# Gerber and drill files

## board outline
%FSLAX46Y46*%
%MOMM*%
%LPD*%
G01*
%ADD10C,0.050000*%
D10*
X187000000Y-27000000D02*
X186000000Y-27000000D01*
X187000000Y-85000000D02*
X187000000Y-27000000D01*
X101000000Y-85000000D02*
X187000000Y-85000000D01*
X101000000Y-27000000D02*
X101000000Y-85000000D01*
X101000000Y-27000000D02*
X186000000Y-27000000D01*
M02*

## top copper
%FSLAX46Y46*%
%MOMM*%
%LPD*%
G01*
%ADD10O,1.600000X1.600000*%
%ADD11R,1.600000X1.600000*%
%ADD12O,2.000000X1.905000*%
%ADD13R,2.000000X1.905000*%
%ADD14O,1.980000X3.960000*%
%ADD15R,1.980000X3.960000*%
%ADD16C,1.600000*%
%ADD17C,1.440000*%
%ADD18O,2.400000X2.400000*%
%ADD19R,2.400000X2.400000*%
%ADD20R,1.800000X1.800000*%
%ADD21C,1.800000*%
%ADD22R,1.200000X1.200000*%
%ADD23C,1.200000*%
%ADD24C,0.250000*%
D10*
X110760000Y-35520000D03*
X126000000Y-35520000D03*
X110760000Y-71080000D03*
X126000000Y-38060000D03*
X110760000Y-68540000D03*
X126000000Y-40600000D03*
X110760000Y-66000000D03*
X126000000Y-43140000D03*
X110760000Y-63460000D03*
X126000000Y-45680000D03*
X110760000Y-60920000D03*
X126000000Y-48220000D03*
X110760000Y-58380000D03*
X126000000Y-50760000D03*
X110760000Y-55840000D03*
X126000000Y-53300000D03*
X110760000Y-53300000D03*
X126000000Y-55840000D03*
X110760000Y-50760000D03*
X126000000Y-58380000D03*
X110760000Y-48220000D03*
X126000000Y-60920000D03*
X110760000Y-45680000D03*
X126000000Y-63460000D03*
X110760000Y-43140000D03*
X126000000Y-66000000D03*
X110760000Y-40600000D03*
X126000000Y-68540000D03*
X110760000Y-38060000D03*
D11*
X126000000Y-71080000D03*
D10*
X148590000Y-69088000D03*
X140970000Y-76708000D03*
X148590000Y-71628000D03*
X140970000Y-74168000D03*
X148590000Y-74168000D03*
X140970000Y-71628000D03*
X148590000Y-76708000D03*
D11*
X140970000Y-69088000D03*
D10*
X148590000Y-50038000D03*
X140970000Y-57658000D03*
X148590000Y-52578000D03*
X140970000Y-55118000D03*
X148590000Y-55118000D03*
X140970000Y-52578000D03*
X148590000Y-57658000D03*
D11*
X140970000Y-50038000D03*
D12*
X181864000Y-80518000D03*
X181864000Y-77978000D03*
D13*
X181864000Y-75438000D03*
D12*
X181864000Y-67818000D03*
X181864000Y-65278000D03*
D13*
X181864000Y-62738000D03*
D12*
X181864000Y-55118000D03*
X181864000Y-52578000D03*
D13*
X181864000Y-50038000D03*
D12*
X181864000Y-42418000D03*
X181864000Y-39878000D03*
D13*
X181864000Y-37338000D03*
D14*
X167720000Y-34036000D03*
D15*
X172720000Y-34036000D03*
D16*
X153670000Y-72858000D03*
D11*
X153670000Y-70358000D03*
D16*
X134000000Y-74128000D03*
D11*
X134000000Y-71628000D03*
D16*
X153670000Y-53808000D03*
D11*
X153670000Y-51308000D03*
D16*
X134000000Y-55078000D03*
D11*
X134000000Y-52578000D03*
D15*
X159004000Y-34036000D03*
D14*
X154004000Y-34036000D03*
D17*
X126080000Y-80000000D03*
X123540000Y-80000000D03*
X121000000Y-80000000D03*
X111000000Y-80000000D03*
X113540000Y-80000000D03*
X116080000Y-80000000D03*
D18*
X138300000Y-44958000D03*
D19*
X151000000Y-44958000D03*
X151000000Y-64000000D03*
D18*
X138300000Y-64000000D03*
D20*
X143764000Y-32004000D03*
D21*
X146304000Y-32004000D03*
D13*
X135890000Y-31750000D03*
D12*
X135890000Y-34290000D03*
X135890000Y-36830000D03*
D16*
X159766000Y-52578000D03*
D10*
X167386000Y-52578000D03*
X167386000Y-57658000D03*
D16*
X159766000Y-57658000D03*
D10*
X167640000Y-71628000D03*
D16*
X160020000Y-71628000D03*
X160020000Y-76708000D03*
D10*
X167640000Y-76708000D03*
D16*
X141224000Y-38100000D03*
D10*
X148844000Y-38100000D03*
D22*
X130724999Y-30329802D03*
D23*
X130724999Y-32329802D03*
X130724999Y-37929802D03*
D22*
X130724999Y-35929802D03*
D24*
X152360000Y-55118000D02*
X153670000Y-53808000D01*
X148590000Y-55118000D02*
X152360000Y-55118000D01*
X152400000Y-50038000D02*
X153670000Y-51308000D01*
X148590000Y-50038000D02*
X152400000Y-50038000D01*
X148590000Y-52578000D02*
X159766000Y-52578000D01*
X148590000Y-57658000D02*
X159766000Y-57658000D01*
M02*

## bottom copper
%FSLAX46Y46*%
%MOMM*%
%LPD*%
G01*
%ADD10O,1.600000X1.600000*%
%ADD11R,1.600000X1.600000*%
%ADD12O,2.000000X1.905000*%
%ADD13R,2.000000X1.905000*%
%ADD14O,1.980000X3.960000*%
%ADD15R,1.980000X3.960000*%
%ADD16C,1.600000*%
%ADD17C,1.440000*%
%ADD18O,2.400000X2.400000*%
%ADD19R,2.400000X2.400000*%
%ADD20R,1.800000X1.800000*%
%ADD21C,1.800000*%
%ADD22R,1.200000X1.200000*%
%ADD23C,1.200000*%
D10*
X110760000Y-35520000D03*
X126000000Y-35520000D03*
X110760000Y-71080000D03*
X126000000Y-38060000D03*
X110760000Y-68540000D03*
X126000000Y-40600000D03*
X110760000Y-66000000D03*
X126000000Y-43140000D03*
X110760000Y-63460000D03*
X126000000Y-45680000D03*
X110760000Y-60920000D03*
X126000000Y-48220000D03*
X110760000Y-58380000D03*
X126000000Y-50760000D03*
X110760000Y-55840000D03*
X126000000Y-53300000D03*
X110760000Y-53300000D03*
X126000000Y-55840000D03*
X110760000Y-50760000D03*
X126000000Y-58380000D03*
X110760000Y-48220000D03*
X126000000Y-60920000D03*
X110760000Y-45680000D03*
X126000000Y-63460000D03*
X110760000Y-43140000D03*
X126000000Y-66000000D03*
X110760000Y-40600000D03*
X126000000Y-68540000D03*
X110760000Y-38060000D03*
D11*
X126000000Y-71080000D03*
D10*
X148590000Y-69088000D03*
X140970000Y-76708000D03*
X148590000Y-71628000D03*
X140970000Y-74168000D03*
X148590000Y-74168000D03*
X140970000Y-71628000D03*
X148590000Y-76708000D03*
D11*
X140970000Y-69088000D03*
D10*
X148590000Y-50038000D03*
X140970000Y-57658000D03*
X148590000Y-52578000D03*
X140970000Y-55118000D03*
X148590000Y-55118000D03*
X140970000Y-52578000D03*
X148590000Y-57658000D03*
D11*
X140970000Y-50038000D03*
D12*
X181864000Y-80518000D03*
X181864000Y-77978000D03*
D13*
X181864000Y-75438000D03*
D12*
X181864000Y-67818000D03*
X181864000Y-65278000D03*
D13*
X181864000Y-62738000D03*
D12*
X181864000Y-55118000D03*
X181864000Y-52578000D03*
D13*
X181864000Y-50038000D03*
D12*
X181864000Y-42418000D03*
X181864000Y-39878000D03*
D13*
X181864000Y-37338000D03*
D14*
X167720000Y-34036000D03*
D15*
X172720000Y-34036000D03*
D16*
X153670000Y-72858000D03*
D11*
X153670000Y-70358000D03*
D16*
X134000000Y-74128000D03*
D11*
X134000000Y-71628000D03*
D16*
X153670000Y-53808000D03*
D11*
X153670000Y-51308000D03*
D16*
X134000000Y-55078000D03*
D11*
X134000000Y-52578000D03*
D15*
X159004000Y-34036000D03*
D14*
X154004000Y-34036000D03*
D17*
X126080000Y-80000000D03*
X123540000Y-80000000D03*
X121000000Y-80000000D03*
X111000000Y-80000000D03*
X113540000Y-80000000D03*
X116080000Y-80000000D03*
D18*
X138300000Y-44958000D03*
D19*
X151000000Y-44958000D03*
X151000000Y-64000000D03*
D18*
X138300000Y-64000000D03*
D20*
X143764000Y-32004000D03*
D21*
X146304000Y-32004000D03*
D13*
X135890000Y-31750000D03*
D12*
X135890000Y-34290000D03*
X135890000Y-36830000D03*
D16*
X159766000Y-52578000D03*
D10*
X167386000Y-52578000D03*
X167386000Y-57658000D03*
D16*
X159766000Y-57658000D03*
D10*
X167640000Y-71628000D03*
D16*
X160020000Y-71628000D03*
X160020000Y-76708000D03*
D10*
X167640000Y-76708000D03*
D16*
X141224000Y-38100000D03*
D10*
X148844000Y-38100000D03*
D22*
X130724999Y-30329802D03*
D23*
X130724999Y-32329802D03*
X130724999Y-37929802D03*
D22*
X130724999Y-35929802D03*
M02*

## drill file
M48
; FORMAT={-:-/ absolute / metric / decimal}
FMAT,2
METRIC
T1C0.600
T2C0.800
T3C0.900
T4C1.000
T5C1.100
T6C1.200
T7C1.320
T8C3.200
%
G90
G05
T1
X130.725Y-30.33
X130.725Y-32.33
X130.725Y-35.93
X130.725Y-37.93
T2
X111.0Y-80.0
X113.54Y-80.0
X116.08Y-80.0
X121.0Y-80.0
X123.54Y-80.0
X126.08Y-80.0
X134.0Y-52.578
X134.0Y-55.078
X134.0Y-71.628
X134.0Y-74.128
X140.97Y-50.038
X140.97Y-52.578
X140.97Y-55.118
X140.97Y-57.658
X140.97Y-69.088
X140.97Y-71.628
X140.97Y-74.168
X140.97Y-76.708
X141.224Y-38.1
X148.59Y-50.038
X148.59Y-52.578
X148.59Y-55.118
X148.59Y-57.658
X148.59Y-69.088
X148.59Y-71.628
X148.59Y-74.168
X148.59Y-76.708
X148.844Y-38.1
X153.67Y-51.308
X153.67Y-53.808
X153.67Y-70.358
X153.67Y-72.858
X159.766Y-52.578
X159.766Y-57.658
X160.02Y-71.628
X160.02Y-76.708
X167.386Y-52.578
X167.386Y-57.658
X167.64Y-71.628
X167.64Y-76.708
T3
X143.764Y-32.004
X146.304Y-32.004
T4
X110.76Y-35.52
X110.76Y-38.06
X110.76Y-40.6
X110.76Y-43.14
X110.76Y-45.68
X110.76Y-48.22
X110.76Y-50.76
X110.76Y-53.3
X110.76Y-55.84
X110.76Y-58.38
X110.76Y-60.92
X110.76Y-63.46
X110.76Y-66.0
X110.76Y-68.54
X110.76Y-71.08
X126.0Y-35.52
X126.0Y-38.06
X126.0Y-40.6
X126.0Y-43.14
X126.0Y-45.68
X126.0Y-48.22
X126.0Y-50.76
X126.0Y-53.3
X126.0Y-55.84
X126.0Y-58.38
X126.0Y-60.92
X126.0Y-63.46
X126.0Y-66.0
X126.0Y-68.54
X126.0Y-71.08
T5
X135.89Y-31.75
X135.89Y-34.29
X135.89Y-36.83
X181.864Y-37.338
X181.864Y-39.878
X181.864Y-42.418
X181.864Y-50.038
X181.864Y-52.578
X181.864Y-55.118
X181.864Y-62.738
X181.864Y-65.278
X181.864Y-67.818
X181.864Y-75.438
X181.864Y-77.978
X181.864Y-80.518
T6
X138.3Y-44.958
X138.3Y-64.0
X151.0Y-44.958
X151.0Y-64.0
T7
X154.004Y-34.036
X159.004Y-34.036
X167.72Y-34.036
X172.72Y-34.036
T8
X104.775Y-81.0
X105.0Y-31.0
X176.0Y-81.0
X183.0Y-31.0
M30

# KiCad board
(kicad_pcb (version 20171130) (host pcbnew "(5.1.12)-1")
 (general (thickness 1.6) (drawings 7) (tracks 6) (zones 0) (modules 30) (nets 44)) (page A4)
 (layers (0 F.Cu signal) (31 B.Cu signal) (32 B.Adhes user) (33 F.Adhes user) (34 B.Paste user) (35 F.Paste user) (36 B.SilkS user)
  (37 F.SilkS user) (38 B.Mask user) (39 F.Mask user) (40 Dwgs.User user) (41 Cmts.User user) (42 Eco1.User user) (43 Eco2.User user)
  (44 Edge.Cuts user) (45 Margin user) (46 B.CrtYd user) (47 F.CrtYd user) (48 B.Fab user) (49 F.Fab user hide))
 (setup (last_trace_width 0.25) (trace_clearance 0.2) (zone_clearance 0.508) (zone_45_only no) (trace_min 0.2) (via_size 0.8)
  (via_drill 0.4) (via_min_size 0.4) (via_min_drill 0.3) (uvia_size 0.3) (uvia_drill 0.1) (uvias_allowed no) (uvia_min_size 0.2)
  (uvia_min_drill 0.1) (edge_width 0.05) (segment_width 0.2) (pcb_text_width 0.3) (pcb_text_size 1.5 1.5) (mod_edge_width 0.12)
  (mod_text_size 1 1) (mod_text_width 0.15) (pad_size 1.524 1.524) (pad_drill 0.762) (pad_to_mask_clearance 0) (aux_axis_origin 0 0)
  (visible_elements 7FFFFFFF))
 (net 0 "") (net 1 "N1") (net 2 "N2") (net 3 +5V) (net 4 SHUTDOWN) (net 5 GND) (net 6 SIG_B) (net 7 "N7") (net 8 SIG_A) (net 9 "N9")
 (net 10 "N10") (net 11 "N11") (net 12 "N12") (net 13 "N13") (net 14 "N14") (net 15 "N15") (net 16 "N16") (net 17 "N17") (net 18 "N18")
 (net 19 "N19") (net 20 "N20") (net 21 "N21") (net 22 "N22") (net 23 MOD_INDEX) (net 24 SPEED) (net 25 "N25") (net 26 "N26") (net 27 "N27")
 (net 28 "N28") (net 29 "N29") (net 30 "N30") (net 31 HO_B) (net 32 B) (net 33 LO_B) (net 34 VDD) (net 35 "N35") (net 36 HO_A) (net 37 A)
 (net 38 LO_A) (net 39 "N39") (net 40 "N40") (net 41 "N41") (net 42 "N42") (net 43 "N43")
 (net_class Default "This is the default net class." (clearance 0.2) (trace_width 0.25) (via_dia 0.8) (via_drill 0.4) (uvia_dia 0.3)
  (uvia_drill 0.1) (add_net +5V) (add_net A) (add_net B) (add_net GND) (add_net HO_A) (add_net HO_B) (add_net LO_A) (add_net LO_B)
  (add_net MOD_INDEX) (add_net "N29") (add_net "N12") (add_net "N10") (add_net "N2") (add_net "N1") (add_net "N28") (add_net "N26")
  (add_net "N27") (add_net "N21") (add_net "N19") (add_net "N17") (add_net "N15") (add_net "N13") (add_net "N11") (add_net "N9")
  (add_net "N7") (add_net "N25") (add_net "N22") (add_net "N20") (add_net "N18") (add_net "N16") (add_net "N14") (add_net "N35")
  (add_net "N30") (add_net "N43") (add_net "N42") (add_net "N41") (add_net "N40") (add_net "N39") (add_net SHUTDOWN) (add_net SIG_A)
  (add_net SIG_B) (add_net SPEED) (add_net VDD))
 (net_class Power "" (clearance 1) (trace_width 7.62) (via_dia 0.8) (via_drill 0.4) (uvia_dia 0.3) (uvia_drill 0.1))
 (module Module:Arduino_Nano (layer F.Cu) (at 126 71.08 180)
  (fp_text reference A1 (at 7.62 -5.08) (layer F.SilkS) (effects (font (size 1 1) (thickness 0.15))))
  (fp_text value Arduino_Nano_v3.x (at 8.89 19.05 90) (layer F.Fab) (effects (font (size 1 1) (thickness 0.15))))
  (pad 16 thru_hole oval (at 15.24 35.56 180) (size 1.6 1.6) (drill 1) (layers *.Cu *.Mask) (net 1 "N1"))
  (pad 15 thru_hole oval (at 0 35.56 180) (size 1.6 1.6) (drill 1) (layers *.Cu *.Mask) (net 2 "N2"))
  (pad 30 thru_hole oval (at 15.24 0 180) (size 1.6 1.6) (drill 1) (layers *.Cu *.Mask) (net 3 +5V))
  (pad 14 thru_hole oval (at 0 33.02 180) (size 1.6 1.6) (drill 1) (layers *.Cu *.Mask) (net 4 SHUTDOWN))
  (pad 29 thru_hole oval (at 15.24 2.54 180) (size 1.6 1.6) (drill 1) (layers *.Cu *.Mask) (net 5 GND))
  (pad 13 thru_hole oval (at 0 30.48 180) (size 1.6 1.6) (drill 1) (layers *.Cu *.Mask) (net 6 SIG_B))
  (pad 28 thru_hole oval (at 15.24 5.08 180) (size 1.6 1.6) (drill 1) (layers *.Cu *.Mask) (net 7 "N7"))
  (pad 12 thru_hole oval (at 0 27.94 180) (size 1.6 1.6) (drill 1) (layers *.Cu *.Mask) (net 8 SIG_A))
  (pad 27 thru_hole oval (at 15.24 7.62 180) (size 1.6 1.6) (drill 1) (layers *.Cu *.Mask) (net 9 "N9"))
  (pad 11 thru_hole oval (at 0 25.4 180) (size 1.6 1.6) (drill 1) (layers *.Cu *.Mask) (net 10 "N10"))
  (pad 26 thru_hole oval (at 15.24 10.16 180) (size 1.6 1.6) (drill 1) (layers *.Cu *.Mask) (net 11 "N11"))
  (pad 10 thru_hole oval (at 0 22.86 180) (size 1.6 1.6) (drill 1) (layers *.Cu *.Mask) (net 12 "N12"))
  (pad 25 thru_hole oval (at 15.24 12.7 180) (size 1.6 1.6) (drill 1) (layers *.Cu *.Mask) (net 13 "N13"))
  (pad 9 thru_hole oval (at 0 20.32 180) (size 1.6 1.6) (drill 1) (layers *.Cu *.Mask) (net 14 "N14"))
  (pad 24 thru_hole oval (at 15.24 15.24 180) (size 1.6 1.6) (drill 1) (layers *.Cu *.Mask) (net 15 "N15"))
  (pad 8 thru_hole oval (at 0 17.78 180) (size 1.6 1.6) (drill 1) (layers *.Cu *.Mask) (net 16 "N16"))
  (pad 23 thru_hole oval (at 15.24 17.78 180) (size 1.6 1.6) (drill 1) (layers *.Cu *.Mask) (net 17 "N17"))
  (pad 7 thru_hole oval (at 0 15.24 180) (size 1.6 1.6) (drill 1) (layers *.Cu *.Mask) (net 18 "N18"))
  (pad 22 thru_hole oval (at 15.24 20.32 180) (size 1.6 1.6) (drill 1) (layers *.Cu *.Mask) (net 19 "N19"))
  (pad 6 thru_hole oval (at 0 12.7 180) (size 1.6 1.6) (drill 1) (layers *.Cu *.Mask) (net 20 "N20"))
  (pad 21 thru_hole oval (at 15.24 22.86 180) (size 1.6 1.6) (drill 1) (layers *.Cu *.Mask) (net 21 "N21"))
  (pad 5 thru_hole oval (at 0 10.16 180) (size 1.6 1.6) (drill 1) (layers *.Cu *.Mask) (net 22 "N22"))
  (pad 20 thru_hole oval (at 15.24 25.4 180) (size 1.6 1.6) (drill 1) (layers *.Cu *.Mask) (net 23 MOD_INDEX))
  (pad 4 thru_hole oval (at 0 7.62 180) (size 1.6 1.6) (drill 1) (layers *.Cu *.Mask) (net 5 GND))
  (pad 19 thru_hole oval (at 15.24 27.94 180) (size 1.6 1.6) (drill 1) (layers *.Cu *.Mask) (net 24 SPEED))
  (pad 3 thru_hole oval (at 0 5.08 180) (size 1.6 1.6) (drill 1) (layers *.Cu *.Mask) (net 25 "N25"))
  (pad 18 thru_hole oval (at 15.24 30.48 180) (size 1.6 1.6) (drill 1) (layers *.Cu *.Mask) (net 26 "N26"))
  (pad 2 thru_hole oval (at 0 2.54 180) (size 1.6 1.6) (drill 1) (layers *.Cu *.Mask) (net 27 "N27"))
  (pad 17 thru_hole oval (at 15.24 33.02 180) (size 1.6 1.6) (drill 1) (layers *.Cu *.Mask) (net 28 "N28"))
  (pad 1 thru_hole rect (at 0 0 180) (size 1.6 1.6) (drill 1) (layers *.Cu *.Mask) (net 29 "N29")))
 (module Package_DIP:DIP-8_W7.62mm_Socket (layer F.Cu) (at 140.97 69.088)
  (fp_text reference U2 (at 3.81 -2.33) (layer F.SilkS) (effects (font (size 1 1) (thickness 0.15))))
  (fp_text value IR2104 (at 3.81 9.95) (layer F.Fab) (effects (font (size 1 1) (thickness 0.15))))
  (pad 8 thru_hole oval (at 7.62 0) (size 1.6 1.6) (drill 0.8) (layers *.Cu *.Mask) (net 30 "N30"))
  (pad 4 thru_hole oval (at 0 7.62) (size 1.6 1.6) (drill 0.8) (layers *.Cu *.Mask) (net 5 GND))
  (pad 7 thru_hole oval (at 7.62 2.54) (size 1.6 1.6) (drill 0.8) (layers *.Cu *.Mask) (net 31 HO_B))
  (pad 3 thru_hole oval (at 0 5.08) (size 1.6 1.6) (drill 0.8) (layers *.Cu *.Mask) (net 4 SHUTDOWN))
  (pad 6 thru_hole oval (at 7.62 5.08) (size 1.6 1.6) (drill 0.8) (layers *.Cu *.Mask) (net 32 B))
  (pad 2 thru_hole oval (at 0 2.54) (size 1.6 1.6) (drill 0.8) (layers *.Cu *.Mask) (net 6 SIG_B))
  (pad 5 thru_hole oval (at 7.62 7.62) (size 1.6 1.6) (drill 0.8) (layers *.Cu *.Mask) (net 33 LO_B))
  (pad 1 thru_hole rect (at 0 0) (size 1.6 1.6) (drill 0.8) (layers *.Cu *.Mask) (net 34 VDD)))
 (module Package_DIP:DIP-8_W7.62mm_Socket (layer F.Cu) (at 140.97 50.038)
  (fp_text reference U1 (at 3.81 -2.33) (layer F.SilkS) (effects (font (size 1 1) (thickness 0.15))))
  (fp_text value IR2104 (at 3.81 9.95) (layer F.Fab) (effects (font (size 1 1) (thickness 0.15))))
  (pad 8 thru_hole oval (at 7.62 0) (size 1.6 1.6) (drill 0.8) (layers *.Cu *.Mask) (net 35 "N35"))
  (pad 4 thru_hole oval (at 0 7.62) (size 1.6 1.6) (drill 0.8) (layers *.Cu *.Mask) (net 5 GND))
  (pad 7 thru_hole oval (at 7.62 2.54) (size 1.6 1.6) (drill 0.8) (layers *.Cu *.Mask) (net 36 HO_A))
  (pad 3 thru_hole oval (at 0 5.08) (size 1.6 1.6) (drill 0.8) (layers *.Cu *.Mask) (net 4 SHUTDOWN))
  (pad 6 thru_hole oval (at 7.62 5.08) (size 1.6 1.6) (drill 0.8) (layers *.Cu *.Mask) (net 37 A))
  (pad 2 thru_hole oval (at 0 2.54) (size 1.6 1.6) (drill 0.8) (layers *.Cu *.Mask) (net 8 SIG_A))
  (pad 5 thru_hole oval (at 7.62 7.62) (size 1.6 1.6) (drill 0.8) (layers *.Cu *.Mask) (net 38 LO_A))
  (pad 1 thru_hole rect (at 0 0) (size 1.6 1.6) (drill 0.8) (layers *.Cu *.Mask) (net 34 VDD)))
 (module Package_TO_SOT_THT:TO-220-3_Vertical (layer F.Cu) (at 181.864 75.438 270)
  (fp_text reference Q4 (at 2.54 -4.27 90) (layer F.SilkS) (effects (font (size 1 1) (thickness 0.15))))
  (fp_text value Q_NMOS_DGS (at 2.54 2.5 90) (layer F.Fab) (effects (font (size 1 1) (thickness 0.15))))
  (pad 3 thru_hole oval (at 5.08 0 270) (size 1.905 2) (drill 1.1) (layers *.Cu *.Mask) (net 5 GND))
  (pad 2 thru_hole oval (at 2.54 0 270) (size 1.905 2) (drill 1.1) (layers *.Cu *.Mask) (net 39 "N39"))
  (pad 1 thru_hole rect (at 0 0 270) (size 1.905 2) (drill 1.1) (layers *.Cu *.Mask) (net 32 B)))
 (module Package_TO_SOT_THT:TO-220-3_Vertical (layer F.Cu) (at 181.864 62.738 270)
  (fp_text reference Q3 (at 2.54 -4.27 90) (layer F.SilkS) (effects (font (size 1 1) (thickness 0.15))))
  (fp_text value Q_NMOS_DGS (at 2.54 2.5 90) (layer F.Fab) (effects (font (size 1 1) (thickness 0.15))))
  (pad 3 thru_hole oval (at 5.08 0 270) (size 1.905 2) (drill 1.1) (layers *.Cu *.Mask) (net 32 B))
  (pad 2 thru_hole oval (at 2.54 0 270) (size 1.905 2) (drill 1.1) (layers *.Cu *.Mask) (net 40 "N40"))
  (pad 1 thru_hole rect (at 0 0 270) (size 1.905 2) (drill 1.1) (layers *.Cu *.Mask) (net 34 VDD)))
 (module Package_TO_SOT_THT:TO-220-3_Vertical (layer F.Cu) (at 181.864 50.038 270)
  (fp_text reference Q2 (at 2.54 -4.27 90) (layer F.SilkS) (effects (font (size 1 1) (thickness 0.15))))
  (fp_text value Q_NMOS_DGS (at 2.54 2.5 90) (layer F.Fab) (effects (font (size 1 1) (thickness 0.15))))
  (pad 3 thru_hole oval (at 5.08 0 270) (size 1.905 2) (drill 1.1) (layers *.Cu *.Mask) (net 5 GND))
  (pad 2 thru_hole oval (at 2.54 0 270) (size 1.905 2) (drill 1.1) (layers *.Cu *.Mask) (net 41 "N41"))
  (pad 1 thru_hole rect (at 0 0 270) (size 1.905 2) (drill 1.1) (layers *.Cu *.Mask) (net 37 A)))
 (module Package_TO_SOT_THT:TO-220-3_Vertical (layer F.Cu) (at 181.864 37.338 270)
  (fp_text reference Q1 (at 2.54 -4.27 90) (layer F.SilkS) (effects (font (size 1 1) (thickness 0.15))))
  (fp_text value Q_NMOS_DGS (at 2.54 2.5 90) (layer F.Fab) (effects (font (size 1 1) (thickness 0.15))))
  (pad 3 thru_hole oval (at 5.08 0 270) (size 1.905 2) (drill 1.1) (layers *.Cu *.Mask) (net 37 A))
  (pad 2 thru_hole oval (at 2.54 0 270) (size 1.905 2) (drill 1.1) (layers *.Cu *.Mask) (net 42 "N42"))
  (pad 1 thru_hole rect (at 0 0 270) (size 1.905 2) (drill 1.1) (layers *.Cu *.Mask) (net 34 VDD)))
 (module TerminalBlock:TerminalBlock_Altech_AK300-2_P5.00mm (layer F.Cu) (at 172.72 34.036 180)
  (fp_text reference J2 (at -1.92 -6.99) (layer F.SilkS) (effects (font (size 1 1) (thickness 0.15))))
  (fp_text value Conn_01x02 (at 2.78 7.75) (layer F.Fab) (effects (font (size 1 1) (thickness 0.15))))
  (pad 2 thru_hole oval (at 5 0 180) (size 1.98 3.96) (drill 1.32) (layers *.Cu *.Mask) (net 32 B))
  (pad 1 thru_hole rect (at 0 0 180) (size 1.98 3.96) (drill 1.32) (layers *.Cu *.Mask) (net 37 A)))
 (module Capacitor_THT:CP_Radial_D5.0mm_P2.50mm (layer F.Cu) (at 153.67 70.358 270)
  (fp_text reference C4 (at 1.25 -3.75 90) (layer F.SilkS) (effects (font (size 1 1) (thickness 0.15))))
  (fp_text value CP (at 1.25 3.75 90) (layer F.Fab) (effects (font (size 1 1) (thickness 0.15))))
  (pad 2 thru_hole circle (at 2.5 0 270) (size 1.6 1.6) (drill 0.8) (layers *.Cu *.Mask) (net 32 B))
  (pad 1 thru_hole rect (at 0 0 270) (size 1.6 1.6) (drill 0.8) (layers *.Cu *.Mask) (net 30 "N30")))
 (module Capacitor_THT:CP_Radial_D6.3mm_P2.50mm (layer F.Cu) (at 134 71.628 270)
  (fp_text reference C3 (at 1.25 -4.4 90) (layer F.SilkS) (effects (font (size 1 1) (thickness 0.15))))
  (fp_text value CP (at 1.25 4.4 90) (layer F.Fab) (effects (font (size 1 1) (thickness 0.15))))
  (pad 2 thru_hole circle (at 2.5 0 270) (size 1.6 1.6) (drill 0.8) (layers *.Cu *.Mask) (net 5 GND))
  (pad 1 thru_hole rect (at 0 0 270) (size 1.6 1.6) (drill 0.8) (layers *.Cu *.Mask) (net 34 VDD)))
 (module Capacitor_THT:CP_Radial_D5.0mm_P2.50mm (layer F.Cu) (at 153.67 51.308 270)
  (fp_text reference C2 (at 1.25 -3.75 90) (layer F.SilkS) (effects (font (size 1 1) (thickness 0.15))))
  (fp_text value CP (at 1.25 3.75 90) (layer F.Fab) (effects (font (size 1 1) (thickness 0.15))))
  (pad 2 thru_hole circle (at 2.5 0 270) (size 1.6 1.6) (drill 0.8) (layers *.Cu *.Mask) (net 37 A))
  (pad 1 thru_hole rect (at 0 0 270) (size 1.6 1.6) (drill 0.8) (layers *.Cu *.Mask) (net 35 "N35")))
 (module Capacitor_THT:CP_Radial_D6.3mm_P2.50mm (layer F.Cu) (at 134 52.578 270)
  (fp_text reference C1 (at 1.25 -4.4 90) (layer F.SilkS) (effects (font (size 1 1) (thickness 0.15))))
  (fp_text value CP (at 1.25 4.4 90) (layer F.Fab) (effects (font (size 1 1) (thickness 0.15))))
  (pad 2 thru_hole circle (at 2.5 0 270) (size 1.6 1.6) (drill 0.8) (layers *.Cu *.Mask) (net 5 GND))
  (pad 1 thru_hole rect (at 0 0 270) (size 1.6 1.6) (drill 0.8) (layers *.Cu *.Mask) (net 34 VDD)))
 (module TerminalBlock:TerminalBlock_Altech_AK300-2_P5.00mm (layer F.Cu) (at 159.004 34.036 180)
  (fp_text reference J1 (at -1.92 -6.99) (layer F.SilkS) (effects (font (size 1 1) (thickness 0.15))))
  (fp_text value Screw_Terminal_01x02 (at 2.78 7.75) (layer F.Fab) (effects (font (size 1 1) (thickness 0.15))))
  (pad 1 thru_hole rect (at 0 0 180) (size 1.98 3.96) (drill 1.32) (layers *.Cu *.Mask) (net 34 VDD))
  (pad 2 thru_hole oval (at 5 0 180) (size 1.98 3.96) (drill 1.32) (layers *.Cu *.Mask) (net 5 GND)))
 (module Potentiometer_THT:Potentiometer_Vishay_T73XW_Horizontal (layer F.Cu) (at 121 80 90)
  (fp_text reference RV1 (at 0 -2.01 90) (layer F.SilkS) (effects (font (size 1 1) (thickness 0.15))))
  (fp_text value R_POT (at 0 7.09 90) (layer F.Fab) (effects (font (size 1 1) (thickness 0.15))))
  (pad 3 thru_hole circle (at 0 5.08 90) (size 1.44 1.44) (drill 0.8) (layers *.Cu *.Mask) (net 5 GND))
  (pad 2 thru_hole circle (at 0 2.54 90) (size 1.44 1.44) (drill 0.8) (layers *.Cu *.Mask) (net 24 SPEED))
  (pad 1 thru_hole circle (at 0 0 90) (size 1.44 1.44) (drill 0.8) (layers *.Cu *.Mask) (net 9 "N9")))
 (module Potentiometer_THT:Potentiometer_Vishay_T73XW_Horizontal (layer F.Cu) (at 111 80 90)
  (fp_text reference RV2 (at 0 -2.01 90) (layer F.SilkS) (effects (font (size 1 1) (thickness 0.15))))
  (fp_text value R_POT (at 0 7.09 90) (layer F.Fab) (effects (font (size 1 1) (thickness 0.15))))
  (pad 1 thru_hole circle (at 0 0 90) (size 1.44 1.44) (drill 0.8) (layers *.Cu *.Mask) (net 9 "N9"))
  (pad 2 thru_hole circle (at 0 2.54 90) (size 1.44 1.44) (drill 0.8) (layers *.Cu *.Mask) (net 23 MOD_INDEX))
  (pad 3 thru_hole circle (at 0 5.08 90) (size 1.44 1.44) (drill 0.8) (layers *.Cu *.Mask) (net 5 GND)))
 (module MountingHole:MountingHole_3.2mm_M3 (layer F.Cu) (at 183 31)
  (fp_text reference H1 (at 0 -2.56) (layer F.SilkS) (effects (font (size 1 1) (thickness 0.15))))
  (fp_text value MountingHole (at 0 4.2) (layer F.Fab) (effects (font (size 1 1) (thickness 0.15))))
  (pad 1 np_thru_hole circle (at 0 0) (size 3.2 3.2) (drill 3.2) (layers *.Cu *.Mask)))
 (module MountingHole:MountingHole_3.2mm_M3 (layer F.Cu) (at 176 81)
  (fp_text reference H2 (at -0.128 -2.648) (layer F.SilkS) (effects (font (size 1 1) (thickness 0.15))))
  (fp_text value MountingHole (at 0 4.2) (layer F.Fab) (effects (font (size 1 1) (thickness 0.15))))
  (pad 1 np_thru_hole circle (at 0 0) (size 3.2 3.2) (drill 3.2) (layers *.Cu *.Mask)))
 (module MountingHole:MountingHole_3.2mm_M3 (layer F.Cu) (at 104.775 81)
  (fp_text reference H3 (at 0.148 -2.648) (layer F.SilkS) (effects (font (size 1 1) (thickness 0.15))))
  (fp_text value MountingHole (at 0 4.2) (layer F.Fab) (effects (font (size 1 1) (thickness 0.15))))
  (pad 1 np_thru_hole circle (at 0 0) (size 3.2 3.2) (drill 3.2) (layers *.Cu *.Mask)))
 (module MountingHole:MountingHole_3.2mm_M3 (layer F.Cu) (at 105 31)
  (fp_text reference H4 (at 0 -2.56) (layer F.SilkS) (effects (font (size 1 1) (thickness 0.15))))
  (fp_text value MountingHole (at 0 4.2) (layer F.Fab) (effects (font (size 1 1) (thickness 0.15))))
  (pad 1 np_thru_hole circle (at 0 0) (size 3.2 3.2) (drill 3.2) (layers *.Cu *.Mask)))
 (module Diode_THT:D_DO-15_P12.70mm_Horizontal (layer F.Cu) (at 151 44.958 180)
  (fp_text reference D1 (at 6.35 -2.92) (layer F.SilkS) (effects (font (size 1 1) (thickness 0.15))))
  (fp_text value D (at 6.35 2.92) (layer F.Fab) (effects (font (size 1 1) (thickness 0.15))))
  (pad 2 thru_hole oval (at 12.7 0 180) (size 2.4 2.4) (drill 1.2) (layers *.Cu *.Mask) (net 34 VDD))
  (pad 1 thru_hole rect (at 0 0 180) (size 2.4 2.4) (drill 1.2) (layers *.Cu *.Mask) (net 35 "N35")))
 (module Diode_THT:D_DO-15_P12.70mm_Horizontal (layer F.Cu) (at 151 64 180)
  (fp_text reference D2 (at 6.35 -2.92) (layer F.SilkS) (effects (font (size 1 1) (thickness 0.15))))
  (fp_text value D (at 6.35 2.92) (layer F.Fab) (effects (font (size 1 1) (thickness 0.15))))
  (pad 1 thru_hole rect (at 0 0 180) (size 2.4 2.4) (drill 1.2) (layers *.Cu *.Mask) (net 30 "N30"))
  (pad 2 thru_hole oval (at 12.7 0 180) (size 2.4 2.4) (drill 1.2) (layers *.Cu *.Mask) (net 34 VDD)))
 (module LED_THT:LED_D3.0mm (layer F.Cu) (at 143.764 32.004)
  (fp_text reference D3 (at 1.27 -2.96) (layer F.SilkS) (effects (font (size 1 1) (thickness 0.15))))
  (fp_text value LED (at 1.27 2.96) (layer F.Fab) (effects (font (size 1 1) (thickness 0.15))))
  (pad 1 thru_hole rect (at 0 0) (size 1.8 1.8) (drill 0.9) (layers *.Cu *.Mask) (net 5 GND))
  (pad 2 thru_hole circle (at 2.54 0) (size 1.8 1.8) (drill 0.9) (layers *.Cu *.Mask) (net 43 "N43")))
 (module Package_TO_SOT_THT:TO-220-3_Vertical (layer F.Cu) (at 135.89 31.75 270)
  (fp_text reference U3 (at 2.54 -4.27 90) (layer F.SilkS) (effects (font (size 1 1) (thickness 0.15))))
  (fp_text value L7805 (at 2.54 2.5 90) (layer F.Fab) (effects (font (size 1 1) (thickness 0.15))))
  (pad 1 thru_hole rect (at 0 0 270) (size 1.905 2) (drill 1.1) (layers *.Cu *.Mask) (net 34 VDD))
  (pad 2 thru_hole oval (at 2.54 0 270) (size 1.905 2) (drill 1.1) (layers *.Cu *.Mask) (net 5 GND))
  (pad 3 thru_hole oval (at 5.08 0 270) (size 1.905 2) (drill 1.1) (layers *.Cu *.Mask) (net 3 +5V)))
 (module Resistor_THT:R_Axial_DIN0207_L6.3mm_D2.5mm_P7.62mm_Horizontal (layer F.Cu) (at 159.766 52.578)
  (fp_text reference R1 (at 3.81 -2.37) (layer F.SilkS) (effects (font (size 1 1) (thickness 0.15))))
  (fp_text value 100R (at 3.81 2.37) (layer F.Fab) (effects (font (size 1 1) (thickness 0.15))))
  (pad 1 thru_hole circle (at 0 0) (size 1.6 1.6) (drill 0.8) (layers *.Cu *.Mask) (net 36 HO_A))
  (pad 2 thru_hole oval (at 7.62 0) (size 1.6 1.6) (drill 0.8) (layers *.Cu *.Mask) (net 42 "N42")))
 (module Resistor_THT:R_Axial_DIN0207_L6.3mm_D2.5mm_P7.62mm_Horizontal (layer F.Cu) (at 159.766 57.658)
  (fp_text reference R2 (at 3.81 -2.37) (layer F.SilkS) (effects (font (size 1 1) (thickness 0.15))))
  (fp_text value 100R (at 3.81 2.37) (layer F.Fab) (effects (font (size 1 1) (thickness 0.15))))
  (pad 2 thru_hole oval (at 7.62 0) (size 1.6 1.6) (drill 0.8) (layers *.Cu *.Mask) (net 41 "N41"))
  (pad 1 thru_hole circle (at 0 0) (size 1.6 1.6) (drill 0.8) (layers *.Cu *.Mask) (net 38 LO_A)))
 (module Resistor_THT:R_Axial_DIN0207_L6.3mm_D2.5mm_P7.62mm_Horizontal (layer F.Cu) (at 160.02 71.628)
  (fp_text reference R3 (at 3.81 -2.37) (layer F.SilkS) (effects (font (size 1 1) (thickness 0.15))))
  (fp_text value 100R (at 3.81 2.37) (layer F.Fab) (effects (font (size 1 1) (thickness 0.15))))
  (pad 2 thru_hole oval (at 7.62 0) (size 1.6 1.6) (drill 0.8) (layers *.Cu *.Mask) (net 40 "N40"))
  (pad 1 thru_hole circle (at 0 0) (size 1.6 1.6) (drill 0.8) (layers *.Cu *.Mask) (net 31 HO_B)))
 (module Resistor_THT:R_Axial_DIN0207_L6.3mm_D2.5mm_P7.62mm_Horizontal (layer F.Cu) (at 160.02 76.708)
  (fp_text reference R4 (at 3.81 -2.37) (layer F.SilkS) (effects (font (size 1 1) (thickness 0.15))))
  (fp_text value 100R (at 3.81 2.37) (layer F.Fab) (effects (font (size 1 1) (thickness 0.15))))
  (pad 1 thru_hole circle (at 0 0) (size 1.6 1.6) (drill 0.8) (layers *.Cu *.Mask) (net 33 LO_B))
  (pad 2 thru_hole oval (at 7.62 0) (size 1.6 1.6) (drill 0.8) (layers *.Cu *.Mask) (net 39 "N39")))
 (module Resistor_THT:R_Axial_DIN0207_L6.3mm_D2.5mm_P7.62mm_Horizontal (layer F.Cu) (at 141.224 38.1)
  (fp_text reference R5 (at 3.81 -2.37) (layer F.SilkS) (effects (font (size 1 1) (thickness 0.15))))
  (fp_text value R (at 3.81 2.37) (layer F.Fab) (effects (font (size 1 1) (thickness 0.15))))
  (pad 1 thru_hole circle (at 0 0) (size 1.6 1.6) (drill 0.8) (layers *.Cu *.Mask) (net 3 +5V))
  (pad 2 thru_hole oval (at 7.62 0) (size 1.6 1.6) (drill 0.8) (layers *.Cu *.Mask) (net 43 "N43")))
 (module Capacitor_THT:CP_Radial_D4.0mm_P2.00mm (layer F.Cu) (at 130.724999 30.329802 270)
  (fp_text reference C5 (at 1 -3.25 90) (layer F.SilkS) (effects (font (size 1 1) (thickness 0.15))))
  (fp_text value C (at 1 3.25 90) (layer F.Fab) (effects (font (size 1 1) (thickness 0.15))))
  (pad 1 thru_hole rect (at 0 0 270) (size 1.2 1.2) (drill 0.6) (layers *.Cu *.Mask) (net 34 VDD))
  (pad 2 thru_hole circle (at 2 0 270) (size 1.2 1.2) (drill 0.6) (layers *.Cu *.Mask) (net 5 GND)))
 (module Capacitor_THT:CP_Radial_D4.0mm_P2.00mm (layer F.Cu) (at 130.724999 35.929802 270)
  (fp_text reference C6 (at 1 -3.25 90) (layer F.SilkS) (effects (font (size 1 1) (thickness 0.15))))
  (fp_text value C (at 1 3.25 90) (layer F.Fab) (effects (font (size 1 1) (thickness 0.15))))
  (pad 2 thru_hole circle (at 2 0 270) (size 1.2 1.2) (drill 0.6) (layers *.Cu *.Mask) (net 5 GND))
  (pad 1 thru_hole rect (at 0 0 270) (size 1.2 1.2) (drill 0.6) (layers *.Cu *.Mask) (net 3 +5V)))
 (gr_line (start 187 27) (end 186 27) (layer Edge.Cuts) (width 0.05))
 (gr_line (start 187 85) (end 187 27) (layer Edge.Cuts) (width 0.05))
 (gr_line (start 101 85) (end 187 85) (layer Edge.Cuts) (width 0.05))
 (gr_line (start 101 27) (end 101 85) (layer Edge.Cuts) (width 0.05))
 (gr_line (start 101 27) (end 186 27) (layer Edge.Cuts) (width 0.05))
 (segment (start 152.36 55.118) (end 153.67 53.808) (width 0.25) (layer F.Cu) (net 37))
 (segment (start 148.59 55.118) (end 152.36 55.118) (width 0.25) (layer F.Cu) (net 37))
 (segment (start 152.4 50.038) (end 153.67 51.308) (width 0.25) (layer F.Cu) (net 35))
 (segment (start 148.59 50.038) (end 152.4 50.038) (width 0.25) (layer F.Cu) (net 35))
 (segment (start 148.59 52.578) (end 159.766 52.578) (width 0.25) (layer F.Cu) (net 36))
 (segment (start 148.59 57.658) (end 159.766 57.658) (width 0.25) (layer F.Cu) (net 38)))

